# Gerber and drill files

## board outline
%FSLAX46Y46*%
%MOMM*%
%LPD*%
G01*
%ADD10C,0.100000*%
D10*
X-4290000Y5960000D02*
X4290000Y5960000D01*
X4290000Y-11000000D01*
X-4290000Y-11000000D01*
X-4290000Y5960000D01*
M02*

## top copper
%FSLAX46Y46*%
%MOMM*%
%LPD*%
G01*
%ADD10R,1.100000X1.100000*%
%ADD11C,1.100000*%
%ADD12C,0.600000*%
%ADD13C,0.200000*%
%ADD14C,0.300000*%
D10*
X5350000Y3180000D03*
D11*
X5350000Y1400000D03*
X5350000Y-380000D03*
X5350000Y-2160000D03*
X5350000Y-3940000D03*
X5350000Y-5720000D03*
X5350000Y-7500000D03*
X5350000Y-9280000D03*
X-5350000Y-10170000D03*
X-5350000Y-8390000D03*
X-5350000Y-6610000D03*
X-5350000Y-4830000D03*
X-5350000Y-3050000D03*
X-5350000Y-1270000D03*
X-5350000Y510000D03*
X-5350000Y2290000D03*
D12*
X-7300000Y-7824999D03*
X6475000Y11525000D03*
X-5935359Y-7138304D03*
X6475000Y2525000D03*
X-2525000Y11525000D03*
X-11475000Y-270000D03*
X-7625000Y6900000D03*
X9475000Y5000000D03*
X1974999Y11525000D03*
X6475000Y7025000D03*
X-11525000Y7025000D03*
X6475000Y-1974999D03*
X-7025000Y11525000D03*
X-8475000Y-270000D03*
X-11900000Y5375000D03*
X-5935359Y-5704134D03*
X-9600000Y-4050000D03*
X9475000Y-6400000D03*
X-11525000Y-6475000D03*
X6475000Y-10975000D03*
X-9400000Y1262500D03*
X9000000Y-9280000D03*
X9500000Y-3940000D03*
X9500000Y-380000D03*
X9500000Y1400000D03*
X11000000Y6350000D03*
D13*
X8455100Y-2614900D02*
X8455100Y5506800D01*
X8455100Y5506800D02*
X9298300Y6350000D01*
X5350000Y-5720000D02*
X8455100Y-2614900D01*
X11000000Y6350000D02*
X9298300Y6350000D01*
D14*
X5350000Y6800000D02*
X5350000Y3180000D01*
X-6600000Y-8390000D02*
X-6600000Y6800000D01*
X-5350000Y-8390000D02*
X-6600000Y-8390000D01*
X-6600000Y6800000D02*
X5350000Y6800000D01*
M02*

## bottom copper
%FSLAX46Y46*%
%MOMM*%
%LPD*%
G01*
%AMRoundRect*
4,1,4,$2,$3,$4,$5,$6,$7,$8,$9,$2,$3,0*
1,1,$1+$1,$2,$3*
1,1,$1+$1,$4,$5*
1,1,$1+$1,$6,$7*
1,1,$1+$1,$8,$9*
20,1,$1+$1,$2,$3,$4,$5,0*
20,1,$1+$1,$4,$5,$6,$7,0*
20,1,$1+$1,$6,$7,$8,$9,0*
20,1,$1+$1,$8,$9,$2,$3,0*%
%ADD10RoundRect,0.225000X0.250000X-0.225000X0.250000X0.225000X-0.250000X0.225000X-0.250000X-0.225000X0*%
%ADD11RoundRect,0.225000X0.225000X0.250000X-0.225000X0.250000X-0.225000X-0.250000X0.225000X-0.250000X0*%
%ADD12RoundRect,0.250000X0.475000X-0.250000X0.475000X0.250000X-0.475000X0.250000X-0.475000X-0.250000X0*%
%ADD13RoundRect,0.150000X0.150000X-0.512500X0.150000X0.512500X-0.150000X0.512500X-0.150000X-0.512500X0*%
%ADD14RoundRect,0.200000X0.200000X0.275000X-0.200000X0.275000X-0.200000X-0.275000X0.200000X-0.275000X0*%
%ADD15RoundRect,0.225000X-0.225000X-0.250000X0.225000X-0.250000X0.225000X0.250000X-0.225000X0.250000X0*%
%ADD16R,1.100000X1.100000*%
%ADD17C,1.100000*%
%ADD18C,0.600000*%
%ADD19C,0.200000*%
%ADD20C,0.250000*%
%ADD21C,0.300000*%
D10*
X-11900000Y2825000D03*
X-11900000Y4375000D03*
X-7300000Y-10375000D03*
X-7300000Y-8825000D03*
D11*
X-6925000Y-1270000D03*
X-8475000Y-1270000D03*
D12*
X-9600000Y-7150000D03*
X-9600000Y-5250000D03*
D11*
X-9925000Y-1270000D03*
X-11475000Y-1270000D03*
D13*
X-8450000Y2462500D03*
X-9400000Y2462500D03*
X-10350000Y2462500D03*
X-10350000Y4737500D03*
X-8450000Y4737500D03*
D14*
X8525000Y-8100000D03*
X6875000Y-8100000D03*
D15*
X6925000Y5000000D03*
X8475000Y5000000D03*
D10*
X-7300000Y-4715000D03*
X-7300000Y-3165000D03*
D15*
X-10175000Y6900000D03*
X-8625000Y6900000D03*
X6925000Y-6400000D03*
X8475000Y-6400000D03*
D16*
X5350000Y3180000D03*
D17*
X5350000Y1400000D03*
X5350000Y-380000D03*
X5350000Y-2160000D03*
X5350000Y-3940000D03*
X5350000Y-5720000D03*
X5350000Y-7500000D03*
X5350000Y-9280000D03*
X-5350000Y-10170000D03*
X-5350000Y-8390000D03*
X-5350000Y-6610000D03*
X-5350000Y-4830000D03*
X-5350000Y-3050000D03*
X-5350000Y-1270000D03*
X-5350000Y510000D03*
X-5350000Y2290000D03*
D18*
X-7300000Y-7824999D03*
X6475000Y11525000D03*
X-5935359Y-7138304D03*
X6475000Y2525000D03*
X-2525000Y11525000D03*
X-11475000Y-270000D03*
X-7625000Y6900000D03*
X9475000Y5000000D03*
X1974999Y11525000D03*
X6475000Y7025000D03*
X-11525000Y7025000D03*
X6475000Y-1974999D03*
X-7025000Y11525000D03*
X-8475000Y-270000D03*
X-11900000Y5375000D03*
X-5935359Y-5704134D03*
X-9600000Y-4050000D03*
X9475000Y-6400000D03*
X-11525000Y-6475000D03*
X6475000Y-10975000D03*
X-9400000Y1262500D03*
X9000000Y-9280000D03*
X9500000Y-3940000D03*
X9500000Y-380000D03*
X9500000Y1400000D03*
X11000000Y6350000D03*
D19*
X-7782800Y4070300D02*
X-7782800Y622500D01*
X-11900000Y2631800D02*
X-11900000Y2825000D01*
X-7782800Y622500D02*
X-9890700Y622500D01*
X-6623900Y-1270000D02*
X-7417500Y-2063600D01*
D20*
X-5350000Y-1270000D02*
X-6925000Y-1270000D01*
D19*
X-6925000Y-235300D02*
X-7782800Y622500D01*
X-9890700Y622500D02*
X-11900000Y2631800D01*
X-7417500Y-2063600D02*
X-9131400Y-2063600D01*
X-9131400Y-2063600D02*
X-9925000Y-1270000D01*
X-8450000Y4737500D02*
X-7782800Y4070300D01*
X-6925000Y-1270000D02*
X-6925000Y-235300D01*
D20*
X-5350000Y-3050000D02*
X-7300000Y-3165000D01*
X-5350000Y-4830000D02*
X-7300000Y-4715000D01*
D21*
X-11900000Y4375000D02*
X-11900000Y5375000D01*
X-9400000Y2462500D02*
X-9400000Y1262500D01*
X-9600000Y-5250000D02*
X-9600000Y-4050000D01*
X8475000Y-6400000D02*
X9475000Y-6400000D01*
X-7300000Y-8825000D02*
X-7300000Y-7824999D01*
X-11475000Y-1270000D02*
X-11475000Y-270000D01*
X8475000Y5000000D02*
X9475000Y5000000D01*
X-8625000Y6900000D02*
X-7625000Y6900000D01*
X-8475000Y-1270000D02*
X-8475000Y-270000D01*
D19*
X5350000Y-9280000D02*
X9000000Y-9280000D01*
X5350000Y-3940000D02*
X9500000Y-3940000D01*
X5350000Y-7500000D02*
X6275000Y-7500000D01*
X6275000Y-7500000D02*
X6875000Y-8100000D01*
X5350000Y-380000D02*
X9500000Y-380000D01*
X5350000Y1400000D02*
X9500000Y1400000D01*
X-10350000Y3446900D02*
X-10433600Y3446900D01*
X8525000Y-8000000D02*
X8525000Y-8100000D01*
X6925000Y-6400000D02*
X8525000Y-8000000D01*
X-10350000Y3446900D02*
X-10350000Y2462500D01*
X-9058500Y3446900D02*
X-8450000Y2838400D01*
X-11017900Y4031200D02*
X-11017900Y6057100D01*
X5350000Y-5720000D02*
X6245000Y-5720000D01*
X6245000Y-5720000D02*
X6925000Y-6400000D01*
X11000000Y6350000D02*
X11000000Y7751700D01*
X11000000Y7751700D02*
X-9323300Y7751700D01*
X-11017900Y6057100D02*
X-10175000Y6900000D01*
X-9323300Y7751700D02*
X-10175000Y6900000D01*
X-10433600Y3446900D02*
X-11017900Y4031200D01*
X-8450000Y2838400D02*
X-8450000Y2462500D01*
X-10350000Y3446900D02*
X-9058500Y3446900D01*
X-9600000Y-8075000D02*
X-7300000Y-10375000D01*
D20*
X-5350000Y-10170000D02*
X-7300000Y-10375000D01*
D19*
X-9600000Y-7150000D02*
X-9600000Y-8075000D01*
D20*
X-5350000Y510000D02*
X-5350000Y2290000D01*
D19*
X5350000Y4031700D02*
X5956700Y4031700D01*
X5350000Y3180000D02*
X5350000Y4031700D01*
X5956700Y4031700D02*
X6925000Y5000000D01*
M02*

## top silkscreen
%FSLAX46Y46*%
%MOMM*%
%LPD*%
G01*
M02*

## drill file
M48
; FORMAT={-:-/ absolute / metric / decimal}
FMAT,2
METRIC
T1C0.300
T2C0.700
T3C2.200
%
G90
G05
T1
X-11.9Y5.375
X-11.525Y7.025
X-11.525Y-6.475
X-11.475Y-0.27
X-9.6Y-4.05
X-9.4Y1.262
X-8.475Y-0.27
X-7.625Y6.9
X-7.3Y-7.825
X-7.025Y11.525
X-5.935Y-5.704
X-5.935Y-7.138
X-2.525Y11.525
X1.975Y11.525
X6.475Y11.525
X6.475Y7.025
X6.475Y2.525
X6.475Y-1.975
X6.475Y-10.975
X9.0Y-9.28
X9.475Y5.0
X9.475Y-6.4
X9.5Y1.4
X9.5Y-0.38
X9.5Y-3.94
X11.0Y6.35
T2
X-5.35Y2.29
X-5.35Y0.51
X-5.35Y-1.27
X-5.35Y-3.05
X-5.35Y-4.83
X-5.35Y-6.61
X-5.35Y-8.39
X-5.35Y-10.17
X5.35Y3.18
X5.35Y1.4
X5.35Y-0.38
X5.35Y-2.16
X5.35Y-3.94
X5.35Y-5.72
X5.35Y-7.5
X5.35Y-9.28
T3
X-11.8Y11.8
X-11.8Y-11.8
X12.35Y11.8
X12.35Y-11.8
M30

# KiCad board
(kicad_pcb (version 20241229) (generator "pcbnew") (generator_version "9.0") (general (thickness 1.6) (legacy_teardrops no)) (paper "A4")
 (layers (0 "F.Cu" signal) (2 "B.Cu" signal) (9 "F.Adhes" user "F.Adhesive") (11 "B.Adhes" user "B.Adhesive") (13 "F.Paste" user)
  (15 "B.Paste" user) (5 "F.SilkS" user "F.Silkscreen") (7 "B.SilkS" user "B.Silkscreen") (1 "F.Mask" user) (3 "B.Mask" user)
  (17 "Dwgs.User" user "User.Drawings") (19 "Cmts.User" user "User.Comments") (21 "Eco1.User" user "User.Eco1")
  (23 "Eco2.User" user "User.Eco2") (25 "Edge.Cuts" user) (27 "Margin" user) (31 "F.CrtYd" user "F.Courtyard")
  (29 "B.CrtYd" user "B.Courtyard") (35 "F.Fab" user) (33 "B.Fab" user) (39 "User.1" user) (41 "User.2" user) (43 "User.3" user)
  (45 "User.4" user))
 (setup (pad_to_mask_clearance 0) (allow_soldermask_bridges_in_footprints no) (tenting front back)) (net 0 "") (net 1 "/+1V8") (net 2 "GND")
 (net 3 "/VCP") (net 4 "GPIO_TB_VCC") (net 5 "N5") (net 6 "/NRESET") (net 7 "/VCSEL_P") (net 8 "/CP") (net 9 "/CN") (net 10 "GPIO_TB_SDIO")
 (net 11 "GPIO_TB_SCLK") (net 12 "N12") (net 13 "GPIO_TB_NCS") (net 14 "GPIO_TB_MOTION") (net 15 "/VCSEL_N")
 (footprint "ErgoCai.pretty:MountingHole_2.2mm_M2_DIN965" (layer "F.Cu") (at 12.35 -11.8)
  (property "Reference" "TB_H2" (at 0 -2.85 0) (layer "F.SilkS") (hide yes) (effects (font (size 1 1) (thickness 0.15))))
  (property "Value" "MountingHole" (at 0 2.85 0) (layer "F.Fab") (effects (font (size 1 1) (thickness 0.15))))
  (pad "" np_thru_hole circle (at 0 0) (size 2.2 2.2) (drill 2.2) (layers "*.Cu" "*.Mask")))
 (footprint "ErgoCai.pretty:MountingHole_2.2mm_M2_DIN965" (layer "F.Cu") (at -11.8 -11.8)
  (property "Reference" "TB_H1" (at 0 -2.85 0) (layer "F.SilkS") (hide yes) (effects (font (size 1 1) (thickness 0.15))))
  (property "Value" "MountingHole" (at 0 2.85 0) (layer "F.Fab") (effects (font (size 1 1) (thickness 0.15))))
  (pad "" np_thru_hole circle (at 0 0) (size 2.2 2.2) (drill 2.2) (layers "*.Cu" "*.Mask")))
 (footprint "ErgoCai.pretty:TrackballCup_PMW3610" (layer "F.Cu") (at 0 0)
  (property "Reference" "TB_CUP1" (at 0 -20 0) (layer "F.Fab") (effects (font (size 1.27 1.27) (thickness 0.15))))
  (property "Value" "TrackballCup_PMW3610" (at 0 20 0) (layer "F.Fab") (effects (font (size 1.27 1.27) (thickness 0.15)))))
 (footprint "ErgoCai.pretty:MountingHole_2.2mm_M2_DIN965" (layer "F.Cu") (at -11.8 11.8)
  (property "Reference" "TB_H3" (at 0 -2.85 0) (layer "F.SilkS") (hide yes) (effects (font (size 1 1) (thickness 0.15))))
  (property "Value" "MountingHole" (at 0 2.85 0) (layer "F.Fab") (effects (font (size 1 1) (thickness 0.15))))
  (pad "" np_thru_hole circle (at 0 0) (size 2.2 2.2) (drill 2.2) (layers "*.Cu" "*.Mask")))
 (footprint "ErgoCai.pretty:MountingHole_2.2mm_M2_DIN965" (layer "F.Cu") (at 12.35 11.8)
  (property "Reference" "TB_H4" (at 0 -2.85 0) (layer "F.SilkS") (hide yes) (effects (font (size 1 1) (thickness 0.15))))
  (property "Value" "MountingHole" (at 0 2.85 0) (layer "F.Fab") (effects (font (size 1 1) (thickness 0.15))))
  (pad "" np_thru_hole circle (at 0 0) (size 2.2 2.2) (drill 2.2) (layers "*.Cu" "*.Mask")))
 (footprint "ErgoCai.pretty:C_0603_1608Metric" (layer "B.Cu") (at -11.9 -3.6 90)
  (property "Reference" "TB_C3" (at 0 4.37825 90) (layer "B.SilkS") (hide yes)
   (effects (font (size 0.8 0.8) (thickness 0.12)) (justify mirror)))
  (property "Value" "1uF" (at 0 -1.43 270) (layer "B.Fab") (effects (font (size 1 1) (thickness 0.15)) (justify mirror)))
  (pad "1" smd roundrect (at -0.775 0 90) (size 0.9 0.95) (layers "B.Cu" "B.Mask" "B.Paste") (roundrect_rratio 0.25) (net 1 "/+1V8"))
  (pad "2" smd roundrect (at 0.775 0 90) (size 0.9 0.95) (layers "B.Cu" "B.Mask" "B.Paste") (roundrect_rratio 0.25) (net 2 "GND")))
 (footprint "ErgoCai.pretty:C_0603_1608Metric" (layer "B.Cu") (at -7.3 9.6 90)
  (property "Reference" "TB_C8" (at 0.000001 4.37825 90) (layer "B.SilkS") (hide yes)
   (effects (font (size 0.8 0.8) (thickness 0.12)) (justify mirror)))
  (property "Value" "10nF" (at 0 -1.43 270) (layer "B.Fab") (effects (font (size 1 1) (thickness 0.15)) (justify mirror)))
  (pad "1" smd roundrect (at -0.775 0 90) (size 0.9 0.95) (layers "B.Cu" "B.Mask" "B.Paste") (roundrect_rratio 0.25) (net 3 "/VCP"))
  (pad "2" smd roundrect (at 0.775 0 90) (size 0.9 0.95) (layers "B.Cu" "B.Mask" "B.Paste") (roundrect_rratio 0.25) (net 2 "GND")))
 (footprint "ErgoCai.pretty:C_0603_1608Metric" (layer "B.Cu") (at -7.7 1.27 180)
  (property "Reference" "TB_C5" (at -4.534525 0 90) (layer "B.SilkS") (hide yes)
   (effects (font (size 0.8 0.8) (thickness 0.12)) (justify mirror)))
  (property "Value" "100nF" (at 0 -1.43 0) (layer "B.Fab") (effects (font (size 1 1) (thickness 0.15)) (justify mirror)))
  (pad "1" smd roundrect (at -0.775 0 180) (size 0.9 0.95) (layers "B.Cu" "B.Mask" "B.Paste") (roundrect_rratio 0.25) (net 1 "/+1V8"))
  (pad "2" smd roundrect (at 0.775 0 180) (size 0.9 0.95) (layers "B.Cu" "B.Mask" "B.Paste") (roundrect_rratio 0.25) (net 2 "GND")))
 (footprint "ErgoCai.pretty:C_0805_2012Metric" (layer "B.Cu") (at -9.6 6.2 90)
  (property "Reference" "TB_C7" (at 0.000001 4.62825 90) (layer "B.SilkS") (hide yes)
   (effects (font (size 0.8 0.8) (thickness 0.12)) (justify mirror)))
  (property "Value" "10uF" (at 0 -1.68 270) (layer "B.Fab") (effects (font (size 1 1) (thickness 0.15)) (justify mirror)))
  (pad "1" smd roundrect (at -0.95 0 90) (size 1 1.45) (layers "B.Cu" "B.Mask" "B.Paste") (roundrect_rratio 0.25) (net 3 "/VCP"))
  (pad "2" smd roundrect (at 0.95 0 90) (size 1 1.45) (layers "B.Cu" "B.Mask" "B.Paste") (roundrect_rratio 0.25) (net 2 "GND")))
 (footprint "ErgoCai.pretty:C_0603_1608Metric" (layer "B.Cu") (at -10.7 1.27 180)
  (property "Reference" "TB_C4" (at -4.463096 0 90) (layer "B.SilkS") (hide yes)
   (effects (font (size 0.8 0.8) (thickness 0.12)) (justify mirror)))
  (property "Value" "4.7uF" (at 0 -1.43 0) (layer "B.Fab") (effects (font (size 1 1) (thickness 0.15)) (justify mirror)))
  (pad "1" smd roundrect (at -0.775 0 180) (size 0.9 0.95) (layers "B.Cu" "B.Mask" "B.Paste") (roundrect_rratio 0.25) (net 1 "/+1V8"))
  (pad "2" smd roundrect (at 0.775 0 180) (size 0.9 0.95) (layers "B.Cu" "B.Mask" "B.Paste") (roundrect_rratio 0.25) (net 2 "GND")))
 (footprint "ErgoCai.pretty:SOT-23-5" (layer "B.Cu") (at -9.4 -3.6 90)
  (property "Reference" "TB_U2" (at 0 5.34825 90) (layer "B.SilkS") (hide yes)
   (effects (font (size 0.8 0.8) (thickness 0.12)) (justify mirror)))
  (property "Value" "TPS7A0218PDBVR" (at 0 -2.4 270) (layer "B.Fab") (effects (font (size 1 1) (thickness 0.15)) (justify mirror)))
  (pad "1" smd roundrect (at -1.1375 0.95 90) (size 1.325 0.6) (layers "B.Cu" "B.Mask" "B.Paste") (roundrect_rratio 0.25)
   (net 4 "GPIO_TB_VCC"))
  (pad "2" smd roundrect (at -1.1375 0 90) (size 1.325 0.6) (layers "B.Cu" "B.Mask" "B.Paste") (roundrect_rratio 0.25) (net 2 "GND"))
  (pad "3" smd roundrect (at -1.1375 -0.95 90) (size 1.325 0.6) (layers "B.Cu" "B.Mask" "B.Paste") (roundrect_rratio 0.25)
   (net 4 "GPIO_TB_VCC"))
  (pad "4" smd roundrect (at 1.1375 -0.95 90) (size 1.325 0.6) (layers "B.Cu" "B.Mask" "B.Paste") (roundrect_rratio 0.25) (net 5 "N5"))
  (pad "5" smd roundrect (at 1.1375 0.95 90) (size 1.325 0.6) (layers "B.Cu" "B.Mask" "B.Paste") (roundrect_rratio 0.25) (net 1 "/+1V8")))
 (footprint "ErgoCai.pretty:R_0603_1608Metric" (layer "B.Cu") (at 7.7 8.1 180)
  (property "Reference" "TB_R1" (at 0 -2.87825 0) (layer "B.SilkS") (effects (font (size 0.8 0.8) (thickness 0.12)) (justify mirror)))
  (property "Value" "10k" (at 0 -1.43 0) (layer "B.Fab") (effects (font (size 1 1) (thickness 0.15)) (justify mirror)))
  (pad "1" smd roundrect (at -0.825 0 180) (size 0.8 0.95) (layers "B.Cu" "B.Mask" "B.Paste") (roundrect_rratio 0.25) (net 4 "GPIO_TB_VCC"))
  (pad "2" smd roundrect (at 0.825 0 180) (size 0.8 0.95) (layers "B.Cu" "B.Mask" "B.Paste") (roundrect_rratio 0.25) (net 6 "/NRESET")))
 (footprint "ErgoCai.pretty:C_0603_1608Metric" (layer "B.Cu") (at 7.7 -5)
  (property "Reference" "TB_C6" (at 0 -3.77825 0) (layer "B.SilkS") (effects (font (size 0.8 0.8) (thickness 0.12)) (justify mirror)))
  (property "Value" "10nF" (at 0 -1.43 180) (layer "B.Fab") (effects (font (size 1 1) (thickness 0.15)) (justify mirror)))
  (pad "1" smd roundrect (at -0.775 0) (size 0.9 0.95) (layers "B.Cu" "B.Mask" "B.Paste") (roundrect_rratio 0.25) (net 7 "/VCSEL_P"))
  (pad "2" smd roundrect (at 0.775 0) (size 0.9 0.95) (layers "B.Cu" "B.Mask" "B.Paste") (roundrect_rratio 0.25) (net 2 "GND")))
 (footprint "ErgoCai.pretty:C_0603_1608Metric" (layer "B.Cu") (at -7.3 3.94 90)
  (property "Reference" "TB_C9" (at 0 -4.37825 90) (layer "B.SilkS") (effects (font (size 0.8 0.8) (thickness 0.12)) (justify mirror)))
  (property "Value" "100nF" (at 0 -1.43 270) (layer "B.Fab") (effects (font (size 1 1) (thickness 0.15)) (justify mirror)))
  (pad "1" smd roundrect (at -0.775 0 90) (size 0.9 0.95) (layers "B.Cu" "B.Mask" "B.Paste") (roundrect_rratio 0.25) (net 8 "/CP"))
  (pad "2" smd roundrect (at 0.775 0 90) (size 0.9 0.95) (layers "B.Cu" "B.Mask" "B.Paste") (roundrect_rratio 0.25) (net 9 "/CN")))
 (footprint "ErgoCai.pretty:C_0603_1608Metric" (layer "B.Cu") (at -9.4 -6.9)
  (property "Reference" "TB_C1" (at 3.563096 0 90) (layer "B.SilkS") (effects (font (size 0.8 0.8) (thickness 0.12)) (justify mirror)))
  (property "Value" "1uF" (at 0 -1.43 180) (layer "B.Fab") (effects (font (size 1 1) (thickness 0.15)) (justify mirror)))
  (pad "1" smd roundrect (at -0.775 0) (size 0.9 0.95) (layers "B.Cu" "B.Mask" "B.Paste") (roundrect_rratio 0.25) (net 4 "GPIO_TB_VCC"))
  (pad "2" smd roundrect (at 0.775 0) (size 0.9 0.95) (layers "B.Cu" "B.Mask" "B.Paste") (roundrect_rratio 0.25) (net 2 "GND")))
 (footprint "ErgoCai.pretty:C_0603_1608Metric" (layer "B.Cu") (at 7.7 6.4)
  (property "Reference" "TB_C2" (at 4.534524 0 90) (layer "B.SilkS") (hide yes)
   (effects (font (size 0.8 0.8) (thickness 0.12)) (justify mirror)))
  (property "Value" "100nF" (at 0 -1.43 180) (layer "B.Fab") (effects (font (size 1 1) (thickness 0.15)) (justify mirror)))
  (pad "1" smd roundrect (at -0.775 0) (size 0.9 0.95) (layers "B.Cu" "B.Mask" "B.Paste") (roundrect_rratio 0.25) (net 4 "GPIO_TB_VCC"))
  (pad "2" smd roundrect (at 0.775 0) (size 0.9 0.95) (layers "B.Cu" "B.Mask" "B.Paste") (roundrect_rratio 0.25) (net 2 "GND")))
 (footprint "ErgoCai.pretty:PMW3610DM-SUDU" (layer "B.Cu") (at 0 0 90)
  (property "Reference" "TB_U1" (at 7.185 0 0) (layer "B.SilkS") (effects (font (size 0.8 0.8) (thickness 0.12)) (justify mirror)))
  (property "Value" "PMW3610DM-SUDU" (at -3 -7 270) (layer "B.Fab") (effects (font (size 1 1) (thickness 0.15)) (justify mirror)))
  (fp_rect (start -11 4.29) (end 5.96 -4.29) (stroke (width 0.1) (type solid)) (fill no) (layer "Edge.Cuts"))
  (pad "1" thru_hole rect (at 3.18 5.35 90) (size 1.1 1.1) (drill 0.7) (layers "*.Cu" "*.Mask") (remove_unused_layers no) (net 7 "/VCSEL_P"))
  (pad "2" thru_hole circle (at 1.4 5.35 90) (size 1.1 1.1) (drill 0.7) (layers "*.Cu" "*.Mask") (remove_unused_layers no)
   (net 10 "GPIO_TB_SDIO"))
  (pad "3" thru_hole circle (at -0.38 5.35 90) (size 1.1 1.1) (drill 0.7) (layers "*.Cu" "*.Mask") (remove_unused_layers no)
   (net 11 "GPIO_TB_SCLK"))
  (pad "4" thru_hole circle (at -2.16 5.35 90) (size 1.1 1.1) (drill 0.7) (layers "*.Cu" "*.Mask") (remove_unused_layers no) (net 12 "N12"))
  (pad "5" thru_hole circle (at -3.94 5.35 90) (size 1.1 1.1) (drill 0.7) (layers "*.Cu" "*.Mask") (remove_unused_layers no)
   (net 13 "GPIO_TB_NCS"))
  (pad "6" thru_hole circle (at -5.72 5.35 90) (size 1.1 1.1) (drill 0.7) (layers "*.Cu" "*.Mask") (remove_unused_layers no)
   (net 4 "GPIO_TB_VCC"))
  (pad "7" thru_hole circle (at -7.5 5.35 90) (size 1.1 1.1) (drill 0.7) (layers "*.Cu" "*.Mask") (remove_unused_layers no)
   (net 6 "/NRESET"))
  (pad "8" thru_hole circle (at -9.28 5.35 90) (size 1.1 1.1) (drill 0.7) (layers "*.Cu" "*.Mask") (remove_unused_layers no)
   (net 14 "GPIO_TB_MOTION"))
  (pad "9" thru_hole circle (at -10.17 -5.35 90) (size 1.1 1.1) (drill 0.7) (layers "*.Cu" "*.Mask") (remove_unused_layers no)
   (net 3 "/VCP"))
  (pad "10" thru_hole circle (at -8.39 -5.35 90) (size 1.1 1.1) (drill 0.7) (layers "*.Cu" "*.Mask") (remove_unused_layers no)
   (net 7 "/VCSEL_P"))
  (pad "11" thru_hole circle (at -6.61 -5.35 90) (size 1.1 1.1) (drill 0.7) (layers "*.Cu" "*.Mask") (remove_unused_layers no) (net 2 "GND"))
  (pad "12" thru_hole circle (at -4.83 -5.35 90) (size 1.1 1.1) (drill 0.7) (layers "*.Cu" "*.Mask") (remove_unused_layers no) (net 8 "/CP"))
  (pad "13" thru_hole circle (at -3.05 -5.35 90) (size 1.1 1.1) (drill 0.7) (layers "*.Cu" "*.Mask") (remove_unused_layers no) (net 9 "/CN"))
  (pad "14" thru_hole circle (at -1.27 -5.35 90) (size 1.1 1.1) (drill 0.7) (layers "*.Cu" "*.Mask") (remove_unused_layers no)
   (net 1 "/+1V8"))
  (pad "15" thru_hole circle (at 0.51 -5.35 90) (size 1.1 1.1) (drill 0.7) (layers "*.Cu" "*.Mask") (remove_unused_layers no)
   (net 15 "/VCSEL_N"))
  (pad "16" thru_hole circle (at 2.29 -5.35 90) (size 1.1 1.1) (drill 0.7) (layers "*.Cu" "*.Mask") (remove_unused_layers no)
   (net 15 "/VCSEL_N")))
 (segment (start -7.7828 -4.0703) (end -7.7828 -0.6225) (width 0.2) (layer "B.Cu") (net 1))
 (segment (start -11.9 -2.6318) (end -11.9 -2.825) (width 0.2) (layer "B.Cu") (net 1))
 (segment (start -7.7828 -0.6225) (end -9.8907 -0.6225) (width 0.2) (layer "B.Cu") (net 1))
 (segment (start -6.6239 1.27) (end -7.4175 2.0636) (width 0.2) (layer "B.Cu") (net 1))
 (segment (start -5.35 1.27) (end -6.925 1.27) (width 0.25) (locked yes) (layer "B.Cu") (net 1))
 (segment (start -6.925 0.2353) (end -7.7828 -0.6225) (width 0.2) (layer "B.Cu") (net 1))
 (segment (start -9.8907 -0.6225) (end -11.9 -2.6318) (width 0.2) (layer "B.Cu") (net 1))
 (segment (start -7.4175 2.0636) (end -9.1314 2.0636) (width 0.2) (layer "B.Cu") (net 1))
 (segment (start -9.1314 2.0636) (end -9.925 1.27) (width 0.2) (layer "B.Cu") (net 1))
 (segment (start -8.45 -4.7375) (end -7.7828 -4.0703) (width 0.2) (layer "B.Cu") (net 1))
 (segment (start -6.925 1.27) (end -6.925 0.2353) (width 0.2) (layer "B.Cu") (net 1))
 (segment (start -5.35 3.05) (end -7.3 3.165) (width 0.25) (locked yes) (layer "B.Cu") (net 9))
 (segment (start -5.35 4.83) (end -7.3 4.715) (width 0.25) (locked yes) (layer "B.Cu") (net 8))
 (via (at -7.3 7.824999) (size 0.6) (drill 0.3) (layers "F.Cu" "B.Cu") (locked yes) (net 2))
 (via (at 6.475 -11.525) (size 0.6) (drill 0.3) (layers "F.Cu" "B.Cu") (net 2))
 (via (at -5.935359 7.138304) (size 0.6) (drill 0.3) (layers "F.Cu" "B.Cu") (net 2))
 (via (at 6.475 -2.525) (size 0.6) (drill 0.3) (layers "F.Cu" "B.Cu") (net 2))
 (via (at -2.525 -11.525) (size 0.6) (drill 0.3) (layers "F.Cu" "B.Cu") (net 2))
 (via (at -11.475 0.27) (size 0.6) (drill 0.3) (layers "F.Cu" "B.Cu") (locked yes) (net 2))
 (via (at -7.625 -6.9) (size 0.6) (drill 0.3) (layers "F.Cu" "B.Cu") (locked yes) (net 2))
 (via (at 9.475 -5) (size 0.6) (drill 0.3) (layers "F.Cu" "B.Cu") (locked yes) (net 2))
 (via (at 1.974999 -11.525) (size 0.6) (drill 0.3) (layers "F.Cu" "B.Cu") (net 2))
 (via (at 6.475 -7.025) (size 0.6) (drill 0.3) (layers "F.Cu" "B.Cu") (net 2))
 (via (at -11.525 -7.025) (size 0.6) (drill 0.3) (layers "F.Cu" "B.Cu") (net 2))
 (via (at 6.475 1.974999) (size 0.6) (drill 0.3) (layers "F.Cu" "B.Cu") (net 2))
 (via (at -7.025 -11.525) (size 0.6) (drill 0.3) (layers "F.Cu" "B.Cu") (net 2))
 (via (at -8.475 0.27) (size 0.6) (drill 0.3) (layers "F.Cu" "B.Cu") (locked yes) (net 2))
 (via (at -11.9 -5.375) (size 0.6) (drill 0.3) (layers "F.Cu" "B.Cu") (locked yes) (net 2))
 (via (at -5.935359 5.704134) (size 0.6) (drill 0.3) (layers "F.Cu" "B.Cu") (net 2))
 (via (at -9.6 4.05) (size 0.6) (drill 0.3) (layers "F.Cu" "B.Cu") (locked yes) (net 2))
 (via (at 9.475 6.4) (size 0.6) (drill 0.3) (layers "F.Cu" "B.Cu") (locked yes) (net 2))
 (via (at -11.525 6.475) (size 0.6) (drill 0.3) (layers "F.Cu" "B.Cu") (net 2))
 (via (at 6.475 10.975) (size 0.6) (drill 0.3) (layers "F.Cu" "B.Cu") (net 2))
 (via (at -9.4 -1.2625) (size 0.6) (drill 0.3) (layers "F.Cu" "B.Cu") (locked yes) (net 2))
 (segment (start -11.9 -4.375) (end -11.9 -5.375) (width 0.3) (locked yes) (layer "B.Cu") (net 2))
 (segment (start -9.4 -2.4625) (end -9.4 -1.2625) (width 0.3) (locked yes) (layer "B.Cu") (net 2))
 (segment (start -9.6 5.25) (end -9.6 4.05) (width 0.3) (locked yes) (layer "B.Cu") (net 2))
 (segment (start 8.475 6.4) (end 9.475 6.4) (width 0.3) (locked yes) (layer "B.Cu") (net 2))
 (segment (start -7.3 8.825) (end -7.3 7.824999) (width 0.3) (locked yes) (layer "B.Cu") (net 2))
 (segment (start -11.475 1.27) (end -11.475 0.27) (width 0.3) (locked yes) (layer "B.Cu") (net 2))
 (segment (start 8.475 -5) (end 9.475 -5) (width 0.3) (locked yes) (layer "B.Cu") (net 2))
 (segment (start -8.625 -6.9) (end -7.625 -6.9) (width 0.3) (locked yes) (layer "B.Cu") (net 2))
 (segment (start -8.475 1.27) (end -8.475 0.27) (width 0.3) (locked yes) (layer "B.Cu") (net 2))
 (via (at 9 9.28) (size 0.6) (drill 0.3) (layers "F.Cu" "B.Cu") (locked yes) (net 14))
 (segment (start 5.35 9.28) (end 9 9.28) (width 0.2) (locked yes) (layer "B.Cu") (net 14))
 (via (at 9.5 3.94) (size 0.6) (drill 0.3) (layers "F.Cu" "B.Cu") (locked yes) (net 13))
 (segment (start 5.35 3.94) (end 9.5 3.94) (width 0.2) (locked yes) (layer "B.Cu") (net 13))
 (segment (start 5.35 7.5) (end 6.275 7.5) (width 0.2) (layer "B.Cu") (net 6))
 (segment (start 6.275 7.5) (end 6.875 8.1) (width 0.2) (layer "B.Cu") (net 6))
 (via (at 9.5 0.38) (size 0.6) (drill 0.3) (layers "F.Cu" "B.Cu") (locked yes) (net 11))
 (segment (start 5.35 0.38) (end 9.5 0.38) (width 0.2) (locked yes) (layer "B.Cu") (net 11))
 (via (at 9.5 -1.4) (size 0.6) (drill 0.3) (layers "F.Cu" "B.Cu") (locked yes) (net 10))
 (segment (start 5.35 -1.4) (end 9.5 -1.4) (width 0.2) (locked yes) (layer "B.Cu") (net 10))
 (segment (start 8.4551 2.6149) (end 8.4551 -5.5068) (width 0.2) (layer "F.Cu") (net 4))
 (segment (start 8.4551 -5.5068) (end 9.2983 -6.35) (width 0.2) (layer "F.Cu") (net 4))
 (segment (start 5.35 5.72) (end 8.4551 2.6149) (width 0.2) (layer "F.Cu") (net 4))
 (segment (start 11 -6.35) (end 9.2983 -6.35) (width 0.2) (layer "F.Cu") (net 4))
 (via (at 11 -6.35) (size 0.6) (drill 0.3) (layers "F.Cu" "B.Cu") (locked yes) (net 4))
 (segment (start -10.35 -3.4469) (end -10.4336 -3.4469) (width 0.2) (layer "B.Cu") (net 4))
 (segment (start 8.525 8) (end 8.525 8.1) (width 0.2) (layer "B.Cu") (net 4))
 (segment (start 6.925 6.4) (end 8.525 8) (width 0.2) (layer "B.Cu") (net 4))
 (segment (start -10.35 -3.4469) (end -10.35 -2.4625) (width 0.2) (layer "B.Cu") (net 4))
 (segment (start -9.0585 -3.4469) (end -8.45 -2.8384) (width 0.2) (layer "B.Cu") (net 4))
 (segment (start -11.0179 -4.0312) (end -11.0179 -6.0571) (width 0.2) (layer "B.Cu") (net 4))
 (segment (start 5.35 5.72) (end 6.245 5.72) (width 0.2) (layer "B.Cu") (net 4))
 (segment (start 6.245 5.72) (end 6.925 6.4) (width 0.2) (layer "B.Cu") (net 4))
 (segment (start 11 -6.35) (end 11 -7.7517) (width 0.2) (layer "B.Cu") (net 4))
 (segment (start 11 -7.7517) (end -9.3233 -7.7517) (width 0.2) (layer "B.Cu") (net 4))
 (segment (start -11.0179 -6.0571) (end -10.175 -6.9) (width 0.2) (layer "B.Cu") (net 4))
 (segment (start -9.3233 -7.7517) (end -10.175 -6.9) (width 0.2) (layer "B.Cu") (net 4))
 (segment (start -10.4336 -3.4469) (end -11.0179 -4.0312) (width 0.2) (layer "B.Cu") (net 4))
 (segment (start -8.45 -2.8384) (end -8.45 -2.4625) (width 0.2) (layer "B.Cu") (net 4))
 (segment (start -10.35 -3.4469) (end -9.0585 -3.4469) (width 0.2) (layer "B.Cu") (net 4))
 (segment (start -9.6 8.075) (end -7.3 10.375) (width 0.2) (layer "B.Cu") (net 3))
 (segment (start -5.35 10.17) (end -7.3 10.375) (width 0.25) (locked yes) (layer "B.Cu") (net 3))
 (segment (start -9.6 7.15) (end -9.6 8.075) (width 0.2) (layer "B.Cu") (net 3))
 (segment (start -5.35 -0.51) (end -5.35 -2.29) (width 0.25) (locked yes) (layer "B.Cu") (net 15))
 (segment (start 5.35 -6.8) (end 5.35 -3.18) (width 0.3) (locked yes) (layer "F.Cu") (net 7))
 (segment (start -6.6 8.39) (end -6.6 -6.8) (width 0.3) (locked yes) (layer "F.Cu") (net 7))
 (segment (start -5.35 8.39) (end -6.6 8.39) (width 0.3) (locked yes) (layer "F.Cu") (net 7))
 (segment (start -6.6 -6.8) (end 5.35 -6.8) (width 0.3) (locked yes) (layer "F.Cu") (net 7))
 (segment (start 5.35 -4.0317) (end 5.9567 -4.0317) (width 0.2) (layer "B.Cu") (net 7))
 (segment (start 5.35 -3.18) (end 5.35 -4.0317) (width 0.2) (layer "B.Cu") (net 7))
 (segment (start 5.9567 -4.0317) (end 6.925 -5) (width 0.2) (layer "B.Cu") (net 7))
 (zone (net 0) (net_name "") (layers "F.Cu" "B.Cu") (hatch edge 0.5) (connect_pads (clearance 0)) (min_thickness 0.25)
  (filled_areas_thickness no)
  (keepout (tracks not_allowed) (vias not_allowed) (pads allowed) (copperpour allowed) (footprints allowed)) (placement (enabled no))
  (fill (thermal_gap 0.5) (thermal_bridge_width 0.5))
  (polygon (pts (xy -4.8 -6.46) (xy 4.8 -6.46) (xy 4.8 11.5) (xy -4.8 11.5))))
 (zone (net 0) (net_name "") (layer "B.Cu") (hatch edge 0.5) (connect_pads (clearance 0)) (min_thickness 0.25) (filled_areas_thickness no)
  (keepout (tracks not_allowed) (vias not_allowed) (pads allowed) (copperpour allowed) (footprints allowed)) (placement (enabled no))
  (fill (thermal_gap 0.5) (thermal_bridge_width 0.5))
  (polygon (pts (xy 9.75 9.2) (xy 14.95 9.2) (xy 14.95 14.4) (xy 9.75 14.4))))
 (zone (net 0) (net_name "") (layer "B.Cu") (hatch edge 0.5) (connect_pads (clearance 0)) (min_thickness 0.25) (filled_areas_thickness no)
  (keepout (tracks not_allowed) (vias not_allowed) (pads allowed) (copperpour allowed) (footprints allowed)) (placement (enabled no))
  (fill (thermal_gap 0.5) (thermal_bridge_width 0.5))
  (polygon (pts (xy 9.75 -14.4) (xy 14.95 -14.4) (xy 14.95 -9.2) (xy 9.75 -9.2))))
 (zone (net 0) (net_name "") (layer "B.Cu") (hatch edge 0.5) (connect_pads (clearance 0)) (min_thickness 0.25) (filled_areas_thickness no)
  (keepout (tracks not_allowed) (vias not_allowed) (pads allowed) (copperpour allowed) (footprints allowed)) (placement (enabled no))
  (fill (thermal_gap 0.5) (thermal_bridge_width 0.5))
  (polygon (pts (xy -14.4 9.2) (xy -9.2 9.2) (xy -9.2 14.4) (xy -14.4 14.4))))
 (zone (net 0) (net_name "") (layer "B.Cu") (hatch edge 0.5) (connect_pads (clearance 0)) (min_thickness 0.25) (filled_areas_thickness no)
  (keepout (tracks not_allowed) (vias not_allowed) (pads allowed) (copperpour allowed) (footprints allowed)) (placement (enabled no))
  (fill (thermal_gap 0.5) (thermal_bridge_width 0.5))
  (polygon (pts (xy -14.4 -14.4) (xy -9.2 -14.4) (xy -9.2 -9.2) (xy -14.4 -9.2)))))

